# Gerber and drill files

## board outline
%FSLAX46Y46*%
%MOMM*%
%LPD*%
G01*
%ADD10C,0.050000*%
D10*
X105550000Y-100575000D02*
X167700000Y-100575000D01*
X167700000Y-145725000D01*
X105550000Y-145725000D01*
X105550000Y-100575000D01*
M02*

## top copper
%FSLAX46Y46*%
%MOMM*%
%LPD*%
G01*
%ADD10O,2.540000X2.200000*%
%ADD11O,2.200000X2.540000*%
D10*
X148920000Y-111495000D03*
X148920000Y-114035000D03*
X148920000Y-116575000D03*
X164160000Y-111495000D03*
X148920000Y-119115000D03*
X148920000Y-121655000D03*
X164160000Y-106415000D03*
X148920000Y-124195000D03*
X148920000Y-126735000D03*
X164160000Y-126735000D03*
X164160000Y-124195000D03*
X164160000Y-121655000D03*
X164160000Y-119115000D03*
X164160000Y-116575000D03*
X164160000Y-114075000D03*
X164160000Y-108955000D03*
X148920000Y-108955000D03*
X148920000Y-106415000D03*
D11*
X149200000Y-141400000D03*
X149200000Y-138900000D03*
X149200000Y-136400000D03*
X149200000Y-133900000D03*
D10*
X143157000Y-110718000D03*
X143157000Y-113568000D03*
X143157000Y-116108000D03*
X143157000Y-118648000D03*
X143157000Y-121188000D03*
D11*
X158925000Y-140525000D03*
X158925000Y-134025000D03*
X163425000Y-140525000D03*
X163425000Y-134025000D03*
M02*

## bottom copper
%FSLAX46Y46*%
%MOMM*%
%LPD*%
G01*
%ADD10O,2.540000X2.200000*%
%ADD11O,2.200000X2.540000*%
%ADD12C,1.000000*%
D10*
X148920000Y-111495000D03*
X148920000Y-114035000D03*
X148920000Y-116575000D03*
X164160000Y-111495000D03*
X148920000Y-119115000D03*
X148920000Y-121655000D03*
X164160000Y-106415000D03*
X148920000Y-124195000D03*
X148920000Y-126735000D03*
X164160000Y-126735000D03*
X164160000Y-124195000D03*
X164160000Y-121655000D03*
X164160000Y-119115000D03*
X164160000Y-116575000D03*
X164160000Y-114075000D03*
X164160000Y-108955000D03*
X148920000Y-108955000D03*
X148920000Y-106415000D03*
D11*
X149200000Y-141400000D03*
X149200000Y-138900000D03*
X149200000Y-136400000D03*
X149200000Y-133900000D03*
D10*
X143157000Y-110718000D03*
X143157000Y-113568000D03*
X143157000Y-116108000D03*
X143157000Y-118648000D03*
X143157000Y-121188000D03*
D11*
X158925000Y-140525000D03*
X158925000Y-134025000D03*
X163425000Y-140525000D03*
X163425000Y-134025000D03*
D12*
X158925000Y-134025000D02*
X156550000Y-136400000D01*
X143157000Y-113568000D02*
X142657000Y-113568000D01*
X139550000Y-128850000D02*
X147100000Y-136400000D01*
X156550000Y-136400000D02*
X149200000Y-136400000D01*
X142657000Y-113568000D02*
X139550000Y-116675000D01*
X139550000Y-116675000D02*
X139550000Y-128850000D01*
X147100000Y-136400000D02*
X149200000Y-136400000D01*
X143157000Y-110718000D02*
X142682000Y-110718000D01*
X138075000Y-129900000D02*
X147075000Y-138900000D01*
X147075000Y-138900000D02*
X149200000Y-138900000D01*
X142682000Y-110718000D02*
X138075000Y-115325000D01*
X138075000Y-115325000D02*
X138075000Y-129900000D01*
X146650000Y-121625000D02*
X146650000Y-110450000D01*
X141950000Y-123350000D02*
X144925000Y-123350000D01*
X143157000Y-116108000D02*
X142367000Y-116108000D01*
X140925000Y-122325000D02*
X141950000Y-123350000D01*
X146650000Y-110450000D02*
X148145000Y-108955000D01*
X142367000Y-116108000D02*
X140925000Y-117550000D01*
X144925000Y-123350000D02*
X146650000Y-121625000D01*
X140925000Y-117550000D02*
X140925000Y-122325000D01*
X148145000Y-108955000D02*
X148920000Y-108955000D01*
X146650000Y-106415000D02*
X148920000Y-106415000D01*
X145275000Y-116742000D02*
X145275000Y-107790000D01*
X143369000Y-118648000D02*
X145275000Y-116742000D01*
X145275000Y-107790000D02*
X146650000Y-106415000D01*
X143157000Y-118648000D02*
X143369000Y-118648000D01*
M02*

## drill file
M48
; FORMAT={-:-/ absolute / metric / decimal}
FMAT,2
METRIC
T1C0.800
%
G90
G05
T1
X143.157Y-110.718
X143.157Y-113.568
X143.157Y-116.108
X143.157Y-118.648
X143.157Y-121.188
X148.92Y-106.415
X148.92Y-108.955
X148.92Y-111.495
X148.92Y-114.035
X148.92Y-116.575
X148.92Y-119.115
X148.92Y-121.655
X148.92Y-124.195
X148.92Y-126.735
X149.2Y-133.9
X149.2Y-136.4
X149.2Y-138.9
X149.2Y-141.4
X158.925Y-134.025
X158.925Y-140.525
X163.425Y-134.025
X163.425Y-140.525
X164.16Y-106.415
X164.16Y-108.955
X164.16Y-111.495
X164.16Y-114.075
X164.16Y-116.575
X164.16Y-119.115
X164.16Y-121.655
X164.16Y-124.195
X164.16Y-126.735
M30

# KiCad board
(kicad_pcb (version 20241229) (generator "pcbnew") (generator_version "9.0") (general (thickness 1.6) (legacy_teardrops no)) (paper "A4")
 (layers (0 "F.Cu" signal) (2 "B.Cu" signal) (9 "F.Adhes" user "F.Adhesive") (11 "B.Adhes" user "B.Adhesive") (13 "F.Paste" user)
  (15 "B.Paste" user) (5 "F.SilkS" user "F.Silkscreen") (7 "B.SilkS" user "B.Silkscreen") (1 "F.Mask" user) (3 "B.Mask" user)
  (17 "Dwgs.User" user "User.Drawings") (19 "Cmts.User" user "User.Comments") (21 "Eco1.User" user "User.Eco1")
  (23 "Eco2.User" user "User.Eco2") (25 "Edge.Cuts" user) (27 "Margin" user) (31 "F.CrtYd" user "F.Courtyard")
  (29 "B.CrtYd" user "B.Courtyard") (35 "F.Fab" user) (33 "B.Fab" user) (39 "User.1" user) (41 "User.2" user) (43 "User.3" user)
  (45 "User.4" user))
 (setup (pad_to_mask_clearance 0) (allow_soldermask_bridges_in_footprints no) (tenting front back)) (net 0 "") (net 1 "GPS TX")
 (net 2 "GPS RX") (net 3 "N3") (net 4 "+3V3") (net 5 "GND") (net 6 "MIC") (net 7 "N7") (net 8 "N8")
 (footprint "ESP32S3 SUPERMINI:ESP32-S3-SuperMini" (layer "F.Cu") (at 156.54 116.575)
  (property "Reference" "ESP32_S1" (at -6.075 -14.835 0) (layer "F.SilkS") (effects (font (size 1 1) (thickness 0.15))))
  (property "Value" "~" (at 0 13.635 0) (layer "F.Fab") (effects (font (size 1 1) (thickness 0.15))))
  (pad "1" thru_hole oval (at -7.62 -5.08) (size 2.54 2.2) (drill 0.8) (layers "*.Cu" "*.Mask") (remove_unused_layers no)
   (thermal_bridge_angle 45))
  (pad "2" thru_hole oval (at -7.62 -2.54) (size 2.54 2.2) (drill 0.8) (layers "*.Cu" "*.Mask") (remove_unused_layers no)
   (thermal_bridge_angle 45))
  (pad "3" thru_hole oval (at -7.62 0) (size 2.54 2.2) (drill 0.8) (layers "*.Cu" "*.Mask") (remove_unused_layers no)
   (thermal_bridge_angle 45))
  (pad "3V3" thru_hole oval (at 7.62 -5.08) (size 2.54 2.2) (drill 0.8) (layers "*.Cu" "*.Mask") (remove_unused_layers no)
   (thermal_bridge_angle 45))
  (pad "4" thru_hole oval (at -7.62 2.54) (size 2.54 2.2) (drill 0.8) (layers "*.Cu" "*.Mask") (remove_unused_layers no)
   (thermal_bridge_angle 45))
  (pad "5" thru_hole oval (at -7.62 5.08) (size 2.54 2.2) (drill 0.8) (layers "*.Cu" "*.Mask") (remove_unused_layers no)
   (thermal_bridge_angle 45))
  (pad "5V" thru_hole oval (at 7.62 -10.16) (size 2.54 2.2) (drill 0.8) (layers "*.Cu" "*.Mask") (remove_unused_layers no)
   (thermal_bridge_angle 45))
  (pad "6" thru_hole oval (at -7.62 7.62) (size 2.54 2.2) (drill 0.8) (layers "*.Cu" "*.Mask") (remove_unused_layers no)
   (thermal_bridge_angle 45))
  (pad "7" thru_hole oval (at -7.62 10.16) (size 2.54 2.2) (drill 0.8) (layers "*.Cu" "*.Mask") (remove_unused_layers no)
   (thermal_bridge_angle 45))
  (pad "8" thru_hole oval (at 7.62 10.16) (size 2.54 2.2) (drill 0.8) (layers "*.Cu" "*.Mask") (remove_unused_layers no)
   (thermal_bridge_angle 45))
  (pad "9" thru_hole oval (at 7.62 7.62) (size 2.54 2.2) (drill 0.8) (layers "*.Cu" "*.Mask") (remove_unused_layers no)
   (thermal_bridge_angle 45))
  (pad "10" thru_hole oval (at 7.62 5.08) (size 2.54 2.2) (drill 0.8) (layers "*.Cu" "*.Mask") (remove_unused_layers no)
   (thermal_bridge_angle 45))
  (pad "11" thru_hole oval (at 7.62 2.54) (size 2.54 2.2) (drill 0.8) (layers "*.Cu" "*.Mask") (remove_unused_layers no)
   (thermal_bridge_angle 45))
  (pad "12" thru_hole oval (at 7.62 0) (size 2.54 2.2) (drill 0.8) (layers "*.Cu" "*.Mask") (remove_unused_layers no)
   (thermal_bridge_angle 45))
  (pad "13" thru_hole oval (at 7.62 -2.5) (size 2.54 2.2) (drill 0.8) (layers "*.Cu" "*.Mask") (remove_unused_layers no)
   (thermal_bridge_angle 45))
  (pad "GND" thru_hole oval (at 7.62 -7.62) (size 2.54 2.2) (drill 0.8) (layers "*.Cu" "*.Mask") (remove_unused_layers no)
   (thermal_bridge_angle 45))
  (pad "RX" thru_hole oval (at -7.62 -7.62) (size 2.54 2.2) (drill 0.8) (layers "*.Cu" "*.Mask") (remove_unused_layers no) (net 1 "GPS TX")
   (thermal_bridge_angle 45))
  (pad "TX" thru_hole oval (at -7.62 -10.16) (size 2.54 2.2) (drill 0.8) (layers "*.Cu" "*.Mask") (remove_unused_layers no) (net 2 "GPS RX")
   (thermal_bridge_angle 45)))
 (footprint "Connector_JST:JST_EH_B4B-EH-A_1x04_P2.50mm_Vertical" (layer "F.Cu") (at 149.2 141.4 90)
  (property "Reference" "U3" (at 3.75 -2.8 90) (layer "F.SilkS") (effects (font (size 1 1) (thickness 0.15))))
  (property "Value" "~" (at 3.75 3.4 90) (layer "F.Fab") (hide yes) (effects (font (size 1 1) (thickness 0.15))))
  (pad "1" thru_hole oval (at 0 0 90) (size 2.54 2.2) (drill 0.8) (layers "*.Cu" "*.Mask") (remove_unused_layers no) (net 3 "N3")
   (thermal_bridge_angle 45))
  (pad "2" thru_hole oval (at 2.5 0 90) (size 2.54 2.2) (drill 0.8) (layers "*.Cu" "*.Mask") (remove_unused_layers no) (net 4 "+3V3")
   (thermal_bridge_angle 45))
  (pad "3" thru_hole oval (at 5 0 90) (size 2.54 2.2) (drill 0.8) (layers "*.Cu" "*.Mask") (remove_unused_layers no) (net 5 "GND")
   (thermal_bridge_angle 45))
  (pad "4" thru_hole oval (at 7.5 0 90) (size 2.54 2.2) (drill 0.8) (layers "*.Cu" "*.Mask") (remove_unused_layers no) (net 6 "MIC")
   (thermal_bridge_angle 45)))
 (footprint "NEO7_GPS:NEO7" (layer "F.Cu") (at 92.738 102.9)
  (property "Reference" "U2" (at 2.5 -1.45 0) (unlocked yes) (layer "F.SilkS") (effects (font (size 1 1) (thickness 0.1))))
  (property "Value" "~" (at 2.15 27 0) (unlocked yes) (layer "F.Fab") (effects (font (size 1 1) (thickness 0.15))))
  (pad "1" thru_hole oval (at 50.419 7.818) (size 2.54 2.2) (drill 0.8) (layers "*.Cu" "*.Mask") (remove_unused_layers no) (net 4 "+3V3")
   (thermal_bridge_angle 45))
  (pad "2" thru_hole oval (at 50.419 10.668) (size 2.54 2.2) (drill 0.8) (layers "*.Cu" "*.Mask") (remove_unused_layers no) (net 5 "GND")
   (thermal_bridge_angle 45))
  (pad "3" thru_hole oval (at 50.419 13.208) (size 2.54 2.2) (drill 0.8) (layers "*.Cu" "*.Mask") (remove_unused_layers no) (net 1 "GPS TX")
   (thermal_bridge_angle 45))
  (pad "4" thru_hole oval (at 50.419 15.748) (size 2.54 2.2) (drill 0.8) (layers "*.Cu" "*.Mask") (remove_unused_layers no) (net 2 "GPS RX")
   (thermal_bridge_angle 45))
  (pad "5" thru_hole oval (at 50.419 18.288) (size 2.54 2.2) (drill 0.8) (layers "*.Cu" "*.Mask") (remove_unused_layers no) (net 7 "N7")
   (thermal_bridge_angle 45)))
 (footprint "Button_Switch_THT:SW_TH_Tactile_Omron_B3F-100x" (layer "F.Cu") (at 158.925 140.525 90)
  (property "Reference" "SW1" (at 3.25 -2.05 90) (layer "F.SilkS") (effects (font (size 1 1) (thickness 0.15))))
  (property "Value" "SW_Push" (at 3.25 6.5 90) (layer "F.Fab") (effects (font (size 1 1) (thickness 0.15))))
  (pad "1" thru_hole oval (at 0 0 90) (size 2.54 2.2) (drill 0.8) (layers "*.Cu" "*.Mask") (remove_unused_layers no) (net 5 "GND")
   (thermal_bridge_angle 45))
  (pad "1" thru_hole oval (at 6.5 0 90) (size 2.54 2.2) (drill 0.8) (layers "*.Cu" "*.Mask") (remove_unused_layers no) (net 5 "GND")
   (thermal_bridge_angle 45))
  (pad "2" thru_hole oval (at 0 4.5 90) (size 2.54 2.2) (drill 0.8) (layers "*.Cu" "*.Mask") (remove_unused_layers no) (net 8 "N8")
   (thermal_bridge_angle 45))
  (pad "2" thru_hole oval (at 6.5 4.5 90) (size 2.54 2.2) (drill 0.8) (layers "*.Cu" "*.Mask") (remove_unused_layers no) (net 8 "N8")
   (thermal_bridge_angle 45)))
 (gr_rect (start 105.55 100.575) (end 167.7 145.725) (stroke (width 0.05) (type default)) (fill no) (layer "Edge.Cuts"))
 (segment (start 158.925 134.025) (end 156.55 136.4) (width 1) (layer "B.Cu") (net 5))
 (segment (start 143.157 113.568) (end 142.657 113.568) (width 1) (layer "B.Cu") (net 5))
 (segment (start 139.55 128.85) (end 147.1 136.4) (width 1) (layer "B.Cu") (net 5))
 (segment (start 156.55 136.4) (end 149.2 136.4) (width 1) (layer "B.Cu") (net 5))
 (segment (start 142.657 113.568) (end 139.55 116.675) (width 1) (layer "B.Cu") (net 5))
 (segment (start 139.55 116.675) (end 139.55 128.85) (width 1) (layer "B.Cu") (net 5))
 (segment (start 147.1 136.4) (end 149.2 136.4) (width 1) (layer "B.Cu") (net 5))
 (segment (start 143.157 110.718) (end 142.682 110.718) (width 1) (layer "B.Cu") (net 4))
 (segment (start 138.075 129.9) (end 147.075 138.9) (width 1) (layer "B.Cu") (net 4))
 (segment (start 147.075 138.9) (end 149.2 138.9) (width 1) (layer "B.Cu") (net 4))
 (segment (start 142.682 110.718) (end 138.075 115.325) (width 1) (layer "B.Cu") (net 4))
 (segment (start 138.075 115.325) (end 138.075 129.9) (width 1) (layer "B.Cu") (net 4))
 (segment (start 146.65 121.625) (end 146.65 110.45) (width 1) (layer "B.Cu") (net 1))
 (segment (start 141.95 123.35) (end 144.925 123.35) (width 1) (layer "B.Cu") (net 1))
 (segment (start 143.157 116.108) (end 142.367 116.108) (width 1) (layer "B.Cu") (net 1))
 (segment (start 140.925 122.325) (end 141.95 123.35) (width 1) (layer "B.Cu") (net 1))
 (segment (start 146.65 110.45) (end 148.145 108.955) (width 1) (layer "B.Cu") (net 1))
 (segment (start 142.367 116.108) (end 140.925 117.55) (width 1) (layer "B.Cu") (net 1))
 (segment (start 144.925 123.35) (end 146.65 121.625) (width 1) (layer "B.Cu") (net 1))
 (segment (start 140.925 117.55) (end 140.925 122.325) (width 1) (layer "B.Cu") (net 1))
 (segment (start 148.145 108.955) (end 148.92 108.955) (width 1) (layer "B.Cu") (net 1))
 (segment (start 146.65 106.415) (end 148.92 106.415) (width 1) (layer "B.Cu") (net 2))
 (segment (start 145.275 116.742) (end 145.275 107.79) (width 1) (layer "B.Cu") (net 2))
 (segment (start 143.369 118.648) (end 145.275 116.742) (width 1) (layer "B.Cu") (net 2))
 (segment (start 145.275 107.79) (end 146.65 106.415) (width 1) (layer "B.Cu") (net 2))
 (segment (start 143.157 118.648) (end 143.369 118.648) (width 1) (layer "B.Cu") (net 2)))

